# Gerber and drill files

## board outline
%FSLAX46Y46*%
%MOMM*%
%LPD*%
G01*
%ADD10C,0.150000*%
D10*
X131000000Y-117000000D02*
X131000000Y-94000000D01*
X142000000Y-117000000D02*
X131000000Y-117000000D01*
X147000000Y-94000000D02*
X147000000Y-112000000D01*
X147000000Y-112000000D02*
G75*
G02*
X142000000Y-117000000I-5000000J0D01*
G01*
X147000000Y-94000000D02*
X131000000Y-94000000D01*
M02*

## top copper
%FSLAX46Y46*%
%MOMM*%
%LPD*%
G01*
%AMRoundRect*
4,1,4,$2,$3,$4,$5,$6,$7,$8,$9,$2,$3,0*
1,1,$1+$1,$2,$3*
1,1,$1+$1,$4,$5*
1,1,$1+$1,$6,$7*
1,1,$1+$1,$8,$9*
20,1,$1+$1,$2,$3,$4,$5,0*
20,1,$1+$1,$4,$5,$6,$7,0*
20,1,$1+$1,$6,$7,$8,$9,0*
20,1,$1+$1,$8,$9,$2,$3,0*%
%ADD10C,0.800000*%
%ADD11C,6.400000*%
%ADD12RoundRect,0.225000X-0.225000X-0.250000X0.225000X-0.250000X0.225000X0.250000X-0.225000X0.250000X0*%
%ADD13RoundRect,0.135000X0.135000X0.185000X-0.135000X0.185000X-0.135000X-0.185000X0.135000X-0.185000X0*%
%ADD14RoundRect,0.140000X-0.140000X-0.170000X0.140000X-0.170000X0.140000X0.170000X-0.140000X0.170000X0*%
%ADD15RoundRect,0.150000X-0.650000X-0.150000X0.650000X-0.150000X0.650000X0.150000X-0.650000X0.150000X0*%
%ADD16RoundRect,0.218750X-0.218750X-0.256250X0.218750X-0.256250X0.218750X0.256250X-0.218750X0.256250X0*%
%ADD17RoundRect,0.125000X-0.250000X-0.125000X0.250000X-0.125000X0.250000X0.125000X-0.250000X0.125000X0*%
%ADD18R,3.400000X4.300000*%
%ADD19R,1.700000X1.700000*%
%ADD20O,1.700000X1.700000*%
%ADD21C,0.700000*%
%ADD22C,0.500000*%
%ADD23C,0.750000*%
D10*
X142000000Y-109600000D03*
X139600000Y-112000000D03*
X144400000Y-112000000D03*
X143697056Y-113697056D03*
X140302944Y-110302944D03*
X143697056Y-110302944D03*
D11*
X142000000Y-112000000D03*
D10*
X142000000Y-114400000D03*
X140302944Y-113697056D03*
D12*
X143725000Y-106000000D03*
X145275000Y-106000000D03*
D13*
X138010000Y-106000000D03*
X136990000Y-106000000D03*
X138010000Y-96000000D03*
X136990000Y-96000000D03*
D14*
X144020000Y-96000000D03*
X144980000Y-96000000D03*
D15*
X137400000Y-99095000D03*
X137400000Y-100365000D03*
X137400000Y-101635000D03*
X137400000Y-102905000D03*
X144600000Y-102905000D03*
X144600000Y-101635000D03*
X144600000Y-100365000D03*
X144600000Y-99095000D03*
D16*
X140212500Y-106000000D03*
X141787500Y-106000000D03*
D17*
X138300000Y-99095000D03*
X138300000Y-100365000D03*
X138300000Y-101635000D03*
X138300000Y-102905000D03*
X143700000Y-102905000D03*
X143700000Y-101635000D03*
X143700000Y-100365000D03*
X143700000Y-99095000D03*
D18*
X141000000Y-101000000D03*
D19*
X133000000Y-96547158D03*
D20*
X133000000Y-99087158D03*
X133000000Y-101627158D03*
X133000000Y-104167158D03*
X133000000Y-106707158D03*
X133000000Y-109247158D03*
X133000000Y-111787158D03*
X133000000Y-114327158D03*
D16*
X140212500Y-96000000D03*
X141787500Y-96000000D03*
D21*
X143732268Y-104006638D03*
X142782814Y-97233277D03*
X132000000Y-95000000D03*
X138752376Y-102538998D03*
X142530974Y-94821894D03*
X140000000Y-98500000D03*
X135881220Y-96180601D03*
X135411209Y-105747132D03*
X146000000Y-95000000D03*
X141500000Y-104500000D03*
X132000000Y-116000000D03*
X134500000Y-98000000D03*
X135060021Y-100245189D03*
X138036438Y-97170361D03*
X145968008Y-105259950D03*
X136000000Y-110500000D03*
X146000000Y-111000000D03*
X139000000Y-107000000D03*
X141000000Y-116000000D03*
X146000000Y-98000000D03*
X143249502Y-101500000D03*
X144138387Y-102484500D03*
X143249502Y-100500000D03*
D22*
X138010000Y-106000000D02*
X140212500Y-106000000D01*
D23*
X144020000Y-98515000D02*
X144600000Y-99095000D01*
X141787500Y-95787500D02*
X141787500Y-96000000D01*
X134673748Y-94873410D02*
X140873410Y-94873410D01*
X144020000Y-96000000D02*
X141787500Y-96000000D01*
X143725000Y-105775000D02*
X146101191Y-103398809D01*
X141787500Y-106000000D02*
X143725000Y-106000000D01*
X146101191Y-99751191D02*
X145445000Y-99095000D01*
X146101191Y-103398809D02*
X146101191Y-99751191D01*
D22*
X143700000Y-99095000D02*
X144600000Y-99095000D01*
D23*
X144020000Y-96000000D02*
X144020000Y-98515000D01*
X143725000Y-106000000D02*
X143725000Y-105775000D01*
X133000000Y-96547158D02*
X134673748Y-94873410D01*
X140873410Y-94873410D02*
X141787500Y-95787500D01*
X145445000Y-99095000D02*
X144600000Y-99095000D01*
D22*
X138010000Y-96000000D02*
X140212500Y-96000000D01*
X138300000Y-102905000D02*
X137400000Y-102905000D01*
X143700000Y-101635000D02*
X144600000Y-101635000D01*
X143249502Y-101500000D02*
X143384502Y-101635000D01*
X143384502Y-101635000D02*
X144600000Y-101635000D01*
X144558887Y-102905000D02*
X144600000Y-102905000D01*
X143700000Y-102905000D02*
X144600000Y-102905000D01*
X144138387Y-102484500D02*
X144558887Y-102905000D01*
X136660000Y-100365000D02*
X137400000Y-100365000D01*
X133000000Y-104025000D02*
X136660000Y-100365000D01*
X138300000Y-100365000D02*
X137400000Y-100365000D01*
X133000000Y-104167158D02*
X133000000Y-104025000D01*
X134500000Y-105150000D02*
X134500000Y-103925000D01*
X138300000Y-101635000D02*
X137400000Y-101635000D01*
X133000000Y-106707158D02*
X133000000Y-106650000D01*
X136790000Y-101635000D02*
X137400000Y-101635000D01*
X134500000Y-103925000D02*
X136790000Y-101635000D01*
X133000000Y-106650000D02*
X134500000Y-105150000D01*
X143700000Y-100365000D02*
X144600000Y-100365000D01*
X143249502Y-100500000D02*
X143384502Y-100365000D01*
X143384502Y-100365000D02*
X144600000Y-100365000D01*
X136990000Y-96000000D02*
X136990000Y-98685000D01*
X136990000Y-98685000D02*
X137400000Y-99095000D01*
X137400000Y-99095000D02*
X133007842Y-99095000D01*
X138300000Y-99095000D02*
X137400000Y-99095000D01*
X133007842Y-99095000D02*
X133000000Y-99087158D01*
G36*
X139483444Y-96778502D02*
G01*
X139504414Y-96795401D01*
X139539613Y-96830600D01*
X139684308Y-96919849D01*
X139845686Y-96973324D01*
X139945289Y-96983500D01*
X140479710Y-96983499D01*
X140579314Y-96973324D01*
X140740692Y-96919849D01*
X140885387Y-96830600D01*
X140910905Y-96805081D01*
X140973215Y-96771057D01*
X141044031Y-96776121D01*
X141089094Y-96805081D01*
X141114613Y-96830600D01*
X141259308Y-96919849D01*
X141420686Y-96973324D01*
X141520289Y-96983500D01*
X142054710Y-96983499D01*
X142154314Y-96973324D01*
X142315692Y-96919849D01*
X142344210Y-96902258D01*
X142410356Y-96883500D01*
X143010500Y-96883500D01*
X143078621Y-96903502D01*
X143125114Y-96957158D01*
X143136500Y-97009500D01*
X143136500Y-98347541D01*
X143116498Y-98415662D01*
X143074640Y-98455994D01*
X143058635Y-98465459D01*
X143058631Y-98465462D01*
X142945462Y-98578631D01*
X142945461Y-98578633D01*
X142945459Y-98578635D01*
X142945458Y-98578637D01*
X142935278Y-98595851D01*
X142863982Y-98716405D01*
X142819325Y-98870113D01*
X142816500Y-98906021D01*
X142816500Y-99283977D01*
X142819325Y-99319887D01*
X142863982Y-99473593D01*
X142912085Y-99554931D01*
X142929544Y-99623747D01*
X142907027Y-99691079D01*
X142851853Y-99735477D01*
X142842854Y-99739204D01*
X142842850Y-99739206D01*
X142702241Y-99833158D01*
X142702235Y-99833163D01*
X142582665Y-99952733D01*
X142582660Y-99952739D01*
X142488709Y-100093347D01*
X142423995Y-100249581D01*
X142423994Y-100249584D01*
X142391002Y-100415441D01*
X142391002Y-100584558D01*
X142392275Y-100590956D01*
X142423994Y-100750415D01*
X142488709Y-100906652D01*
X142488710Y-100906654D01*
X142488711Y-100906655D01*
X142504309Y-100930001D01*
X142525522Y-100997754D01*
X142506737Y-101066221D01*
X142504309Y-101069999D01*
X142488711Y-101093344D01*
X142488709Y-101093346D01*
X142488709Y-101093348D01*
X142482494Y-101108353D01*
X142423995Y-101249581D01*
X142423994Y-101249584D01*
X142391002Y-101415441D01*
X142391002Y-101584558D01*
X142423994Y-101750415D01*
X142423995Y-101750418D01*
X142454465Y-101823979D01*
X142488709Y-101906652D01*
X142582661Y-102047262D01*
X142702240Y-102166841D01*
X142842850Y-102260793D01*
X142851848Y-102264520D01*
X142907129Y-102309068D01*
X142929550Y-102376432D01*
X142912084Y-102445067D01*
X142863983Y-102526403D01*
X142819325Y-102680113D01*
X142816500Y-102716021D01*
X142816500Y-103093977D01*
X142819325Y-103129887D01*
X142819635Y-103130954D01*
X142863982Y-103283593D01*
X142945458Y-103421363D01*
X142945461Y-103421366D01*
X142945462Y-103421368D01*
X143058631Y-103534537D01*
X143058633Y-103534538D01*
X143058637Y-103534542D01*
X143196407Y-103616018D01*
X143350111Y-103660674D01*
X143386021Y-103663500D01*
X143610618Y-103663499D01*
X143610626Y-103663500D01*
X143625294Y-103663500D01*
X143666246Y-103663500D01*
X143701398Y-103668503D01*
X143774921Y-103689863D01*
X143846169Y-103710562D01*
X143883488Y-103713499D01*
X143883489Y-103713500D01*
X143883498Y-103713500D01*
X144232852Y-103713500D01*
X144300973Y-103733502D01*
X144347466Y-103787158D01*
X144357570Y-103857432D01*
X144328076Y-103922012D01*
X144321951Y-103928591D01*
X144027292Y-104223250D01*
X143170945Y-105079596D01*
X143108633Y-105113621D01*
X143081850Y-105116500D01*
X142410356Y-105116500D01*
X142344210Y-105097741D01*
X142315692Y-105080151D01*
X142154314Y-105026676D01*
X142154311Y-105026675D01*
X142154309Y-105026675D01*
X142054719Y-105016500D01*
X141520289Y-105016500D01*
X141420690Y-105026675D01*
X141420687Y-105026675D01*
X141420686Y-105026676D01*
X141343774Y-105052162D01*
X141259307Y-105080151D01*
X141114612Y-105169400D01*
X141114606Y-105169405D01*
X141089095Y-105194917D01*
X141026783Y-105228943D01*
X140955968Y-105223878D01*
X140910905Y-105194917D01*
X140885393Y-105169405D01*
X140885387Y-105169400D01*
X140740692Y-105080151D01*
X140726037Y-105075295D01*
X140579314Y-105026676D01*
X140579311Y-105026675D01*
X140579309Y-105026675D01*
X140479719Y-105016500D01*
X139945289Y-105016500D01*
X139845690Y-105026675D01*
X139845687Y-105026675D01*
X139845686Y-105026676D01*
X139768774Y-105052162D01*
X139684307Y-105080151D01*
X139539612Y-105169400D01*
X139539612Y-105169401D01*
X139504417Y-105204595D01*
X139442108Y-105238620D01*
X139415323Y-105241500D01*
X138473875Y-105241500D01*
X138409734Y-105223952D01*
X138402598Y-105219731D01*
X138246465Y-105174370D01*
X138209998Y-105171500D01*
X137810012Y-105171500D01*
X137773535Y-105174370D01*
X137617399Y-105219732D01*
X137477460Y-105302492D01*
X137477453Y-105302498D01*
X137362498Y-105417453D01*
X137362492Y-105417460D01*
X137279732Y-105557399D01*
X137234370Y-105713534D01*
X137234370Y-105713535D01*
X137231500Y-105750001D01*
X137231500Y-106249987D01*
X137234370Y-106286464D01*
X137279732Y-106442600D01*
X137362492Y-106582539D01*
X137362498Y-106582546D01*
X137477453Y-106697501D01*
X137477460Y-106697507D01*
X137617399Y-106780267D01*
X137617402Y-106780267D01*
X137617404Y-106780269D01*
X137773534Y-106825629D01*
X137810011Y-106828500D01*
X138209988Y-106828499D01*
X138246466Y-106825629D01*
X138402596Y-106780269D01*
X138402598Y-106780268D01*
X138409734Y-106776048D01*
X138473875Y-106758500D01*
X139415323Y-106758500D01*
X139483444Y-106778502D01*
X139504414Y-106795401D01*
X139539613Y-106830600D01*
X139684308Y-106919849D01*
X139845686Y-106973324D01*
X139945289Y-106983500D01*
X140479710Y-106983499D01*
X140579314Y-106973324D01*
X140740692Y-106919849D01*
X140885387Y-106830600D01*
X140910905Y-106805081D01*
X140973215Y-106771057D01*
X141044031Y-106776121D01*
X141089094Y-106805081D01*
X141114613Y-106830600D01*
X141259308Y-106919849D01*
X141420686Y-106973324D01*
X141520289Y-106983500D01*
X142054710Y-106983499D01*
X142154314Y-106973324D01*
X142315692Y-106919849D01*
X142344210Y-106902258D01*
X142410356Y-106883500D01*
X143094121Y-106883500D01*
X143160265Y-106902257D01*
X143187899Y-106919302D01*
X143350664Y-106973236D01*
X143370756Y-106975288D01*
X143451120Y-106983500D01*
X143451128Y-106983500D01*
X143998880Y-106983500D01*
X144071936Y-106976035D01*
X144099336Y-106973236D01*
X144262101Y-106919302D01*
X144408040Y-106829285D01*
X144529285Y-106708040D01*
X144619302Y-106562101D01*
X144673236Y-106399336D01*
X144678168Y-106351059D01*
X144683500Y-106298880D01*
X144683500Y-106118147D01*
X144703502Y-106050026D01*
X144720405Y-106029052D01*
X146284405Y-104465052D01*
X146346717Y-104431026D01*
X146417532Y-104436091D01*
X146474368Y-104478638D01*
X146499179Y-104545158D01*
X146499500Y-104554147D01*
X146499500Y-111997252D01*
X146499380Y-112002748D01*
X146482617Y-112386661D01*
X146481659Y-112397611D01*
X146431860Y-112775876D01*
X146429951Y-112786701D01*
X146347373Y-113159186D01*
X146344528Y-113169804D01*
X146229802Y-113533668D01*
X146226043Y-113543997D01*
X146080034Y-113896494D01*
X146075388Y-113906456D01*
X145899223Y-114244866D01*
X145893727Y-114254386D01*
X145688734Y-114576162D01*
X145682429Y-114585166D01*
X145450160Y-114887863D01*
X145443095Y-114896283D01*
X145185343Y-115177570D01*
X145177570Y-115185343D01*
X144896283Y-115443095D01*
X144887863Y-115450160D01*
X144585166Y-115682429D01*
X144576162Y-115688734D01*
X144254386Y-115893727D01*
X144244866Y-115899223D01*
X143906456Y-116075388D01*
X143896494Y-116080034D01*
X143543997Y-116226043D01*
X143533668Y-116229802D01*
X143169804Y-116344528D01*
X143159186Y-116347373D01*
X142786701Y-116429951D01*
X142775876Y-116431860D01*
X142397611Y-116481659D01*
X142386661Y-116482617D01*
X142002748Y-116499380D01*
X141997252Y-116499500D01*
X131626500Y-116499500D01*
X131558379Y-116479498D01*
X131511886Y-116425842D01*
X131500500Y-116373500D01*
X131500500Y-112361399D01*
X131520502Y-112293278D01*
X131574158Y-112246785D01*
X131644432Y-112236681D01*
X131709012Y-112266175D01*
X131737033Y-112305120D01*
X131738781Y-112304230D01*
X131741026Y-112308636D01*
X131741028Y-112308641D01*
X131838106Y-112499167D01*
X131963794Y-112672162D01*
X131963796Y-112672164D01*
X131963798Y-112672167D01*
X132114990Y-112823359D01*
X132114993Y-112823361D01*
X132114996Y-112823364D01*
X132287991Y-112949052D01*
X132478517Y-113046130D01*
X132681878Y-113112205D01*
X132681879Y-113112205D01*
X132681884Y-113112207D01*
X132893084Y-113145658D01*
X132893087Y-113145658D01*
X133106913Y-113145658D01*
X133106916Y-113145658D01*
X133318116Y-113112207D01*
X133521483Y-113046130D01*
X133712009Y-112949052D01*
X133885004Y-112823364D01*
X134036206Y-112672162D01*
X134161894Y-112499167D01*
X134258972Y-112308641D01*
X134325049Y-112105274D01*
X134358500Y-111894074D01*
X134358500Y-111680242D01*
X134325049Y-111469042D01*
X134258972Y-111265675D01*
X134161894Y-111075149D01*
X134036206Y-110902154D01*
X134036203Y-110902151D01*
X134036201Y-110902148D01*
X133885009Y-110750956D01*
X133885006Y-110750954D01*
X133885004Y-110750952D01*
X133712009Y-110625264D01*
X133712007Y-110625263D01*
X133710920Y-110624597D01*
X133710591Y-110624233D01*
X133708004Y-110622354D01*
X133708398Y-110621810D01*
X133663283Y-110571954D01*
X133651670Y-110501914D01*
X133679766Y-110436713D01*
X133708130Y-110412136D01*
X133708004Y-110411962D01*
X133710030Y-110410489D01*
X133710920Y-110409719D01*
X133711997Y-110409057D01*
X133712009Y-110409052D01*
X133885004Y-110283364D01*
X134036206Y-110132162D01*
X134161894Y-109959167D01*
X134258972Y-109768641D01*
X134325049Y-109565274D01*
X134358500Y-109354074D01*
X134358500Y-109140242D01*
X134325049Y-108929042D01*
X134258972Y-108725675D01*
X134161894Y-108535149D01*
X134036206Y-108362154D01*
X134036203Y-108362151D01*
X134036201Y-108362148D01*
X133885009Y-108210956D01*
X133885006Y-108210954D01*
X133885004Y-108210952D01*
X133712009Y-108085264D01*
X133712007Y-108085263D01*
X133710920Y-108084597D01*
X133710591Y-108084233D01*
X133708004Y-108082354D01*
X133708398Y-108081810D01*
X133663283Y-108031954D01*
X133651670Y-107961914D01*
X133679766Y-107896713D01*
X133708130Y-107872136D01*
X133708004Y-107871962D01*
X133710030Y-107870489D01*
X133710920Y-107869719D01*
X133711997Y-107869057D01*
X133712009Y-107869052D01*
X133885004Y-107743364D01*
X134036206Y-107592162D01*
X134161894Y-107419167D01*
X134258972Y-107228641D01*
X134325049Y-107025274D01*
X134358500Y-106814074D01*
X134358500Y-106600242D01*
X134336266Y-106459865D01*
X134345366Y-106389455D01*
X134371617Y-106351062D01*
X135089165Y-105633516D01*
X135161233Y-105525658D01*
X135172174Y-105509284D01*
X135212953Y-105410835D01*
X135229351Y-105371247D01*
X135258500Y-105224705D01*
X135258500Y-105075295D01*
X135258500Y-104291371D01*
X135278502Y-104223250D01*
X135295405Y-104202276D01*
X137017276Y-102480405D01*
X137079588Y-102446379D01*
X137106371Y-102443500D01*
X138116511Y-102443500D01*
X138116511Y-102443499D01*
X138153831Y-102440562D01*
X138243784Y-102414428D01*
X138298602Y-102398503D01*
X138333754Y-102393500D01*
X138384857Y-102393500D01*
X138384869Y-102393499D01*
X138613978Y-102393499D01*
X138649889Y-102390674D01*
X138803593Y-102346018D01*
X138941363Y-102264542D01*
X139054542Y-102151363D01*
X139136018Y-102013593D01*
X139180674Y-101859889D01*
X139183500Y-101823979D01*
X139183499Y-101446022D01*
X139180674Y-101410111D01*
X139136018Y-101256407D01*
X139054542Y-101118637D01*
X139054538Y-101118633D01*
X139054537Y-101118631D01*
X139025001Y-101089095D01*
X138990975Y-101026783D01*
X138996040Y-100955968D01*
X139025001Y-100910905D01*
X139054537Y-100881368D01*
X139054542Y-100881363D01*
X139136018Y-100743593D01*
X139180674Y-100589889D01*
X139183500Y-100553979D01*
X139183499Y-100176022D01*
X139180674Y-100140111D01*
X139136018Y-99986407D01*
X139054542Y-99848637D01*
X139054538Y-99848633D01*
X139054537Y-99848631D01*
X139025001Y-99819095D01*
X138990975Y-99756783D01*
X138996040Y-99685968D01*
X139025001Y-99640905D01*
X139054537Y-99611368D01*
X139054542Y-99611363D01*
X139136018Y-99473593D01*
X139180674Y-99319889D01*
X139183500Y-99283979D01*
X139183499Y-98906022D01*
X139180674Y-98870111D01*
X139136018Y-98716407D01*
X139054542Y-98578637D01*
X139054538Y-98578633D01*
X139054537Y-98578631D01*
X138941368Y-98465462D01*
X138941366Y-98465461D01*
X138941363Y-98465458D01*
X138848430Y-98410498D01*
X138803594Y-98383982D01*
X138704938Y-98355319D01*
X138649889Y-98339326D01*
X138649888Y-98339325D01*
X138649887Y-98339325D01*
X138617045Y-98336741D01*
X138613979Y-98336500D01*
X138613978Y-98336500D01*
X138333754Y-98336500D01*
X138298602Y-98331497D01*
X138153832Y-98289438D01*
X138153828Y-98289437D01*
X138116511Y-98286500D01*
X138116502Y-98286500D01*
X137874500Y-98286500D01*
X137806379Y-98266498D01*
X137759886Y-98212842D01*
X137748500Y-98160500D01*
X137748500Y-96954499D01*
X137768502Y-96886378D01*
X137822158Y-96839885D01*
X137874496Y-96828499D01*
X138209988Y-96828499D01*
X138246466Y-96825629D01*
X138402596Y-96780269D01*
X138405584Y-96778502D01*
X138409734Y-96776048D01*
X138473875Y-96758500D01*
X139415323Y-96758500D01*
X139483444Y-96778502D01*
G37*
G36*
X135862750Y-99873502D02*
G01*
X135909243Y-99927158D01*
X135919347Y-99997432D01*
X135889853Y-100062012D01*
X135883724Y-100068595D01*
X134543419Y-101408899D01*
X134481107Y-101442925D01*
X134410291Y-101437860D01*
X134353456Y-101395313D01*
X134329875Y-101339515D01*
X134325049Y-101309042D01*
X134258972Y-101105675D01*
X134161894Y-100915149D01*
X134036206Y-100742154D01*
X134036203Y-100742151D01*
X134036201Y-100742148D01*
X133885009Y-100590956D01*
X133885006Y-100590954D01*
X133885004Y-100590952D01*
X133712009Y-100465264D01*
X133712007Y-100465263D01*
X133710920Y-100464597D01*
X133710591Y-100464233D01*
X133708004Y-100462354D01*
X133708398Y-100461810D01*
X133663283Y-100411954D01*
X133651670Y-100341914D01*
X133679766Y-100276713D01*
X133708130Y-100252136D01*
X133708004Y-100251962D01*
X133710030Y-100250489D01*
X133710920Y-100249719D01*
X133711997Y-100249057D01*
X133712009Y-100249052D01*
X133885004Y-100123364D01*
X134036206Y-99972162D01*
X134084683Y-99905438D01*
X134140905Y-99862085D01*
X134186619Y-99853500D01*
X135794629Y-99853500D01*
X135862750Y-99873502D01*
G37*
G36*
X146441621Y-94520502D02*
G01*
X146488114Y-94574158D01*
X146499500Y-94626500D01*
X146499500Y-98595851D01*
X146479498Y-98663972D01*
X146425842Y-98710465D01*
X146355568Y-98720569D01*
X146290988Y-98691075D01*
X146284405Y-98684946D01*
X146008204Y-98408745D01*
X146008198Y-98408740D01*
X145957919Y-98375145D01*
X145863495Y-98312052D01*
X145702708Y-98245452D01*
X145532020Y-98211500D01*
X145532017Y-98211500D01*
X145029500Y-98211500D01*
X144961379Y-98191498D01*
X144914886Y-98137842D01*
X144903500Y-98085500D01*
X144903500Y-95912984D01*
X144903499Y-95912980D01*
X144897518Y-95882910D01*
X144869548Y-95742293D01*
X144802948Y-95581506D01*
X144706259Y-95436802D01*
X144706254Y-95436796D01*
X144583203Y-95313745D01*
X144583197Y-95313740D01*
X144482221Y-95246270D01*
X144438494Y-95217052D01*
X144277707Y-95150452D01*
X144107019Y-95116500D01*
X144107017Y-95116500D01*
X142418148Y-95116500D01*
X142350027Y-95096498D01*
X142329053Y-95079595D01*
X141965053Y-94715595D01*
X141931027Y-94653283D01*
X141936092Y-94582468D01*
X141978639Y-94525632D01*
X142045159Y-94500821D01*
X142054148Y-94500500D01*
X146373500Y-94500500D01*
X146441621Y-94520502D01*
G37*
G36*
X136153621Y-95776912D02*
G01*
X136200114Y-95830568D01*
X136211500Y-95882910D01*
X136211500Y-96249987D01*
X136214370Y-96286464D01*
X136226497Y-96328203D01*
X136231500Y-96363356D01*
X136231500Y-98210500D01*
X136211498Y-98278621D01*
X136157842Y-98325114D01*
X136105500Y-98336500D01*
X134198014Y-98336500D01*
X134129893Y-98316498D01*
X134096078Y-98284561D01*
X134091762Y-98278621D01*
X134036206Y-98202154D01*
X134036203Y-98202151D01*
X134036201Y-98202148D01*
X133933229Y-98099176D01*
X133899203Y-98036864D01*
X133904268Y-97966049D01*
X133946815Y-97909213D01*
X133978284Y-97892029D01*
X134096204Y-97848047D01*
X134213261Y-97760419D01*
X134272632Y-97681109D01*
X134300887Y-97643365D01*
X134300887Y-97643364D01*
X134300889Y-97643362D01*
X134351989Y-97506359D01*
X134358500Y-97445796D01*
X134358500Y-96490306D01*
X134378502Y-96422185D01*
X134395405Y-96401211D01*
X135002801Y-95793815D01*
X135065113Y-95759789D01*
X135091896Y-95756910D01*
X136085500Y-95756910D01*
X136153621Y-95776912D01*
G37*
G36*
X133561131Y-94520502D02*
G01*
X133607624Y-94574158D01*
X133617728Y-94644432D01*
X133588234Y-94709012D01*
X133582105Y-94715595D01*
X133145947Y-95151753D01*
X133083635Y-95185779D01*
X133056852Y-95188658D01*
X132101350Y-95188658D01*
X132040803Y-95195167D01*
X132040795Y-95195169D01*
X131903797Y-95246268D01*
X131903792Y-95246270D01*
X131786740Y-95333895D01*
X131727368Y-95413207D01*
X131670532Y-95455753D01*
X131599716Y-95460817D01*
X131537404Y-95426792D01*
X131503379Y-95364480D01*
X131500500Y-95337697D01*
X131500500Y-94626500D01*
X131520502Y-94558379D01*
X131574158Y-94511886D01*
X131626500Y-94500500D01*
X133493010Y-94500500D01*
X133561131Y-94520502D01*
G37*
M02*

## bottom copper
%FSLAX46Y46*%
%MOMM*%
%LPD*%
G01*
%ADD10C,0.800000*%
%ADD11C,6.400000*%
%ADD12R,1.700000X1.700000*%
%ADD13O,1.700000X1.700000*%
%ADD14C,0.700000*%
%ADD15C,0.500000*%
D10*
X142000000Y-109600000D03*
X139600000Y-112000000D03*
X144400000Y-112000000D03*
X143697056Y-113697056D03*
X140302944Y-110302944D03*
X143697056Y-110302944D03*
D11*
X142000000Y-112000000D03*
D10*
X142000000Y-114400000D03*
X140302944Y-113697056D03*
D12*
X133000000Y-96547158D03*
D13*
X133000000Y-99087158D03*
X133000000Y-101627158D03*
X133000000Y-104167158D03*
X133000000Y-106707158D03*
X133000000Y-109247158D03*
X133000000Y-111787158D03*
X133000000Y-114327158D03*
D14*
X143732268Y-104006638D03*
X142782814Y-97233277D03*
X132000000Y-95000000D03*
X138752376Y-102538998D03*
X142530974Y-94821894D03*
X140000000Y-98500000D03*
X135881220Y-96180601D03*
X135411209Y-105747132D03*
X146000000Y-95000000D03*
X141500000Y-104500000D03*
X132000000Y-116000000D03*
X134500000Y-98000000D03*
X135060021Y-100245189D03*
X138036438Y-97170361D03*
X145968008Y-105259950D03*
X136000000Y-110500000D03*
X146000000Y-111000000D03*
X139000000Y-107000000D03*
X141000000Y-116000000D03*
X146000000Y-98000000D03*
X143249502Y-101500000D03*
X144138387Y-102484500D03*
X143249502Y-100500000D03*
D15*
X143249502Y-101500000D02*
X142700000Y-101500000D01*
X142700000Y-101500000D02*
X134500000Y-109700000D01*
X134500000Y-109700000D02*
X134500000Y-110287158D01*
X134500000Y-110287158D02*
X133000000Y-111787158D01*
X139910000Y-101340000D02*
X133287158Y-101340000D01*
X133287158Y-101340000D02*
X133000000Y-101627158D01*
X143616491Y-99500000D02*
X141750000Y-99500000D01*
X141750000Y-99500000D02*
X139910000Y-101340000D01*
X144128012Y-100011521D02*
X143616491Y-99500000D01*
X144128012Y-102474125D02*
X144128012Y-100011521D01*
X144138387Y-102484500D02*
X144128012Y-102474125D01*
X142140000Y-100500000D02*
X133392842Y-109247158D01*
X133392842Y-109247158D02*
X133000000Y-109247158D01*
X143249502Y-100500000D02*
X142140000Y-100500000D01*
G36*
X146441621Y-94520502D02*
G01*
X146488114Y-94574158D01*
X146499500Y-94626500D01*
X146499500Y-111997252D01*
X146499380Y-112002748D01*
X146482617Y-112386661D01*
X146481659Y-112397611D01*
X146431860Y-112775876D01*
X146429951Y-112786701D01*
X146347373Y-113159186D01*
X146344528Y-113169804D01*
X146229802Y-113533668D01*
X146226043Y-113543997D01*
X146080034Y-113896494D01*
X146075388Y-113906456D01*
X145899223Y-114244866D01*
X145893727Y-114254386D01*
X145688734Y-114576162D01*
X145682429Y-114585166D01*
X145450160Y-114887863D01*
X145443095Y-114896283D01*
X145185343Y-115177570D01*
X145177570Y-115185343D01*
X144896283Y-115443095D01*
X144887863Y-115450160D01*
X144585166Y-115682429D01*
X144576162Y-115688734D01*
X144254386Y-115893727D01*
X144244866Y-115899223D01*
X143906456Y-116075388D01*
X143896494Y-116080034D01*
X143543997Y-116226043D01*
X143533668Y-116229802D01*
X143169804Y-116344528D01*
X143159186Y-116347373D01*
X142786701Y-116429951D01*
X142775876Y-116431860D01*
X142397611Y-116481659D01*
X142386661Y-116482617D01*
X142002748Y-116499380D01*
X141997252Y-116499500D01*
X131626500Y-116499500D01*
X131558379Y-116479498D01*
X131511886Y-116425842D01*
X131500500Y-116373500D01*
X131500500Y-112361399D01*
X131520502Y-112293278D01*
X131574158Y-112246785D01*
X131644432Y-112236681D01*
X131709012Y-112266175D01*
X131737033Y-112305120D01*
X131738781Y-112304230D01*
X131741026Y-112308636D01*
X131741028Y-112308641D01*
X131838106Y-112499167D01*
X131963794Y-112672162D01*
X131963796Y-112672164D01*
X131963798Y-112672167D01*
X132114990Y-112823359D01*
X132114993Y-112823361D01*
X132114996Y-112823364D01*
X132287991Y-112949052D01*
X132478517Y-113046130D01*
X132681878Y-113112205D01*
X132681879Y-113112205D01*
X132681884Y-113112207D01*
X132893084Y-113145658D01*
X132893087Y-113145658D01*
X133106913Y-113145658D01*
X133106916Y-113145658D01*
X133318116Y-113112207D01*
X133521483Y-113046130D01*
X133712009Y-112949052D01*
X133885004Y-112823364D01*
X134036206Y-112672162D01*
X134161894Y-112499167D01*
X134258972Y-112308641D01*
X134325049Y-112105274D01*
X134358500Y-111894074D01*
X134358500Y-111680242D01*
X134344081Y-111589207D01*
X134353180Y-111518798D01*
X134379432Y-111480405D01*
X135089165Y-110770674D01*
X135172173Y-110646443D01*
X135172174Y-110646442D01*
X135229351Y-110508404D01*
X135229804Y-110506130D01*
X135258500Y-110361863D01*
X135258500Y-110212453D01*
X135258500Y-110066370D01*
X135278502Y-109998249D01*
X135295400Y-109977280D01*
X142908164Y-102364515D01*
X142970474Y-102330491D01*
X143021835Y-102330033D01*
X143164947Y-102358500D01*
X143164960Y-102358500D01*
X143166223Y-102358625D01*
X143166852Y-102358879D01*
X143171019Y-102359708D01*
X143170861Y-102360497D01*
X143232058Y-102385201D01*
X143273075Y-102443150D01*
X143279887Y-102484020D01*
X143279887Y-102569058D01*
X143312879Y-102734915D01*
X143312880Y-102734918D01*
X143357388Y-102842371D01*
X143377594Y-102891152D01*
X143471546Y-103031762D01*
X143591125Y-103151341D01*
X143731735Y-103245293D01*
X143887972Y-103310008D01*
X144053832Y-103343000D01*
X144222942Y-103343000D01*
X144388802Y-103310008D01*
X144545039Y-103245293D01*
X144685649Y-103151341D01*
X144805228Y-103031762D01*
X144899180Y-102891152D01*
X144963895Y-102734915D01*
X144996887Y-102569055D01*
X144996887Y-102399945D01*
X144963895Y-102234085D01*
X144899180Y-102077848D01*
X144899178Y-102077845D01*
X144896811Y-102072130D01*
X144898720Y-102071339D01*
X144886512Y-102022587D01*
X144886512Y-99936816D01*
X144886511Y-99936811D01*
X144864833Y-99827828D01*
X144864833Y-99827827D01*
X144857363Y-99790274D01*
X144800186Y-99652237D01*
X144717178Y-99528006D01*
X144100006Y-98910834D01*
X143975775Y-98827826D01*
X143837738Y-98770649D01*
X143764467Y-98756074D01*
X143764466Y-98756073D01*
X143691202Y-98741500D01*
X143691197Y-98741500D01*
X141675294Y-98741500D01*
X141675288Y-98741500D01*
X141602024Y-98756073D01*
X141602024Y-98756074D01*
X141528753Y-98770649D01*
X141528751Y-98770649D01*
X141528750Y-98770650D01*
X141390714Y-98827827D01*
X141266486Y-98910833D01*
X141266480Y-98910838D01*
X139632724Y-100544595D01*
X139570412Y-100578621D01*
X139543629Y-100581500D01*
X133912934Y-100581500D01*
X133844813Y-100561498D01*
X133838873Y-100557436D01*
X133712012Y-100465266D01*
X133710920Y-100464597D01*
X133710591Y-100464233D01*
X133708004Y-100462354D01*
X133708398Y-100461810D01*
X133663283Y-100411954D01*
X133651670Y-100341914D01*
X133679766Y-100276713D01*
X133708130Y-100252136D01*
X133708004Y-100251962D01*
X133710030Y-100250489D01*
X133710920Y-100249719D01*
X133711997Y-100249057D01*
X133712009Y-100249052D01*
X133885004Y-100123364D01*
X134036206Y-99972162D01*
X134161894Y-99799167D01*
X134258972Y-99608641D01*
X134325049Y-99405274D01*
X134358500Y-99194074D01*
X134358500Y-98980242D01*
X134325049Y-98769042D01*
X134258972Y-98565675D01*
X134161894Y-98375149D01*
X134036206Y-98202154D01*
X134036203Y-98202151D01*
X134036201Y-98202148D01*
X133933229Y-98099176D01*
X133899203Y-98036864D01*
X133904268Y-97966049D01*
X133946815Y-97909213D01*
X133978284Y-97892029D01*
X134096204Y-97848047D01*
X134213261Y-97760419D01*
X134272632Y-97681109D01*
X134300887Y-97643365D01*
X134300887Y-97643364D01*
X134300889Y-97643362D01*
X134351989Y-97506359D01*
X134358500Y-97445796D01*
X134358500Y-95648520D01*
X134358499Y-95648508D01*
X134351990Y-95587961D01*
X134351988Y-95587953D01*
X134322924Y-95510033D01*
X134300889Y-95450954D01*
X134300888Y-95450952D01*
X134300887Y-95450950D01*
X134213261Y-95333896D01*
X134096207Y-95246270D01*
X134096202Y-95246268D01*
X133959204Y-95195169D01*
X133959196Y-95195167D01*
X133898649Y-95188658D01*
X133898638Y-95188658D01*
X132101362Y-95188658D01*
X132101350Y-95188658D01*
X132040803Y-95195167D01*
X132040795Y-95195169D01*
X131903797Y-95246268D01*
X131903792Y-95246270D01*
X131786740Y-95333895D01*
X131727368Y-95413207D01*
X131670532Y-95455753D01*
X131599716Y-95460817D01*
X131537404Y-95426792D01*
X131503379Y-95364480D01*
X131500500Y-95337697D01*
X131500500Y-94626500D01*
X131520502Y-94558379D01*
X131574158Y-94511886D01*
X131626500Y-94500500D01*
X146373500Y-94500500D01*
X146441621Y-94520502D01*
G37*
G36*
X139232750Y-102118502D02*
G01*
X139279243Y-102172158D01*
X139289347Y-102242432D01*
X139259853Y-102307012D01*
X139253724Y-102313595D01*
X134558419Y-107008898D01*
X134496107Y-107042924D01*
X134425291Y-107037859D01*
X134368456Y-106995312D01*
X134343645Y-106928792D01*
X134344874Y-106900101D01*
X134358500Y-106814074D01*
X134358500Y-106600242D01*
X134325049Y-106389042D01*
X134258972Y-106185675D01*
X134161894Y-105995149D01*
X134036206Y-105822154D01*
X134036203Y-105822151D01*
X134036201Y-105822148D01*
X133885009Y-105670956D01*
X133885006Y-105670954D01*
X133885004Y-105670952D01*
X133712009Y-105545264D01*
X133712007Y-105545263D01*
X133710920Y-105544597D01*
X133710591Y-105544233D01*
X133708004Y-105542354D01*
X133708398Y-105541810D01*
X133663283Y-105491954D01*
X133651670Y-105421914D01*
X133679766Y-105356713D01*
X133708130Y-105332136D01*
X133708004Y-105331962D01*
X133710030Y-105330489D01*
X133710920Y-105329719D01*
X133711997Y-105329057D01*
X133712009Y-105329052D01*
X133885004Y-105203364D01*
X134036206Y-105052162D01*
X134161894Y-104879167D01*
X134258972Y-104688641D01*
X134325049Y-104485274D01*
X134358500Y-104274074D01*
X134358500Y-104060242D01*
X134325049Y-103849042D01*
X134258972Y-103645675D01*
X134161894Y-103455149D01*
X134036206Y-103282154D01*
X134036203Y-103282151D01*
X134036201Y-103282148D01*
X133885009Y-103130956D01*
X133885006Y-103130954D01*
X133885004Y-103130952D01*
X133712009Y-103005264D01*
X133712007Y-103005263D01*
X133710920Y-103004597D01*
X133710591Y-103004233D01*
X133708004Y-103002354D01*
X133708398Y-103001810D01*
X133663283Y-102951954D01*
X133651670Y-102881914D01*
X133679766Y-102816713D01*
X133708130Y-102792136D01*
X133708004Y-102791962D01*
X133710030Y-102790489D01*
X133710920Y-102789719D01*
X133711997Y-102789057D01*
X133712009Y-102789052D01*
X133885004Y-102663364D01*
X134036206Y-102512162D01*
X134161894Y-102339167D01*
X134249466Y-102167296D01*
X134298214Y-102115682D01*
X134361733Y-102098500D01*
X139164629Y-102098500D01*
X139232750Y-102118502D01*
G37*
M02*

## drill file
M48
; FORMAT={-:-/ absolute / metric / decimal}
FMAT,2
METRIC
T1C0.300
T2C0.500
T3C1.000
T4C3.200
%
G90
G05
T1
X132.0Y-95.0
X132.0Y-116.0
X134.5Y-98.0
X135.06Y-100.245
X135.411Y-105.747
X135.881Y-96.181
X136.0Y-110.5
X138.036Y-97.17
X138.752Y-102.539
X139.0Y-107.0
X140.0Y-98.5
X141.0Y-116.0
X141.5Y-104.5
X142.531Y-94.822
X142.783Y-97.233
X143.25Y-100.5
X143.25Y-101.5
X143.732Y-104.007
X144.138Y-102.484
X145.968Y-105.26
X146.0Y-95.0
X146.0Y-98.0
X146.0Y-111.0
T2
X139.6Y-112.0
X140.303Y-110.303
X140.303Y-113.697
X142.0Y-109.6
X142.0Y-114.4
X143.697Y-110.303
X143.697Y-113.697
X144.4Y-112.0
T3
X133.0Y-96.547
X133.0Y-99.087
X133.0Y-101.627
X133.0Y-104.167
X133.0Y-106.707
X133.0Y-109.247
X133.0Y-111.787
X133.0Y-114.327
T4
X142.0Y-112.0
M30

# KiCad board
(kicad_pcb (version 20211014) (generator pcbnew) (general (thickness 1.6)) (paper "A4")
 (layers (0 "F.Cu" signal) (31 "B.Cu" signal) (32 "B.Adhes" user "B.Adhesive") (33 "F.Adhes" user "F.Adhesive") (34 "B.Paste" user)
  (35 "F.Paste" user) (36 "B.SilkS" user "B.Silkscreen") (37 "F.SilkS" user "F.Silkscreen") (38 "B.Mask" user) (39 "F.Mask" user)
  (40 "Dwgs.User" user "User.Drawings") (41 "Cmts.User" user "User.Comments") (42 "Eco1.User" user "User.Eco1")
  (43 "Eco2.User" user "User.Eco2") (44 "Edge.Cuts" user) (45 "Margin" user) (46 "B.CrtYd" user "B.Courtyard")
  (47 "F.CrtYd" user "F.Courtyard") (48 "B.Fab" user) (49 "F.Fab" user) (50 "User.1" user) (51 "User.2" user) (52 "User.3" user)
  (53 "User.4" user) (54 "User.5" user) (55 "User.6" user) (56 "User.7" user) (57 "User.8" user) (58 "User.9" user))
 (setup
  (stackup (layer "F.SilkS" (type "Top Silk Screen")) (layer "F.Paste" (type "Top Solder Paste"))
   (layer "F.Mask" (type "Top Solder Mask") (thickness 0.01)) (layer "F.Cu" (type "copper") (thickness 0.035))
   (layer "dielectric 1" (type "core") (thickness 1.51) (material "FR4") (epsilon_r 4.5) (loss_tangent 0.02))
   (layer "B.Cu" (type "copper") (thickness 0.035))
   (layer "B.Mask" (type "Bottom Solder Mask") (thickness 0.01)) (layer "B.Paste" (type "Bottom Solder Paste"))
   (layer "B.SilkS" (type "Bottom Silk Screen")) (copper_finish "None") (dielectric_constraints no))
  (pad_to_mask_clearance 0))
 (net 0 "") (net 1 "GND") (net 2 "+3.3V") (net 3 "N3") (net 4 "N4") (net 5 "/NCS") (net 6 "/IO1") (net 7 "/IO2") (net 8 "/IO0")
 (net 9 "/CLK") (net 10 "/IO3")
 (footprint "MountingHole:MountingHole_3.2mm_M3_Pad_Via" (layer "F.Cu") (at 142 112)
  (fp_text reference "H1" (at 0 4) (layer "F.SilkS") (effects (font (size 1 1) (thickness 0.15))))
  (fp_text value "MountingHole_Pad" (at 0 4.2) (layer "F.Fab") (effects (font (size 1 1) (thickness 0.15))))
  (pad "1" thru_hole circle (at 0 -2.4) (size 0.8 0.8) (drill 0.5) (layers *.Cu *.Mask) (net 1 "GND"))
  (pad "1" thru_hole circle (at -2.4 0) (size 0.8 0.8) (drill 0.5) (layers *.Cu *.Mask) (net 1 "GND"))
  (pad "1" thru_hole circle (at 2.4 0) (size 0.8 0.8) (drill 0.5) (layers *.Cu *.Mask) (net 1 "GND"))
  (pad "1" thru_hole circle (at 1.697056 1.697056) (size 0.8 0.8) (drill 0.5) (layers *.Cu *.Mask) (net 1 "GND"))
  (pad "1" thru_hole circle (at -1.697056 -1.697056) (size 0.8 0.8) (drill 0.5) (layers *.Cu *.Mask) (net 1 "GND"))
  (pad "1" thru_hole circle (at 1.697056 -1.697056) (size 0.8 0.8) (drill 0.5) (layers *.Cu *.Mask) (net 1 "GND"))
  (pad "1" thru_hole circle (at 0 0) (size 6.4 6.4) (drill 3.2) (layers *.Cu *.Mask) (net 1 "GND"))
  (pad "1" thru_hole circle (at 0 2.4) (size 0.8 0.8) (drill 0.5) (layers *.Cu *.Mask) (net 1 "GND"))
  (pad "1" thru_hole circle (at -1.697056 1.697056) (size 0.8 0.8) (drill 0.5) (layers *.Cu *.Mask) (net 1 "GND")))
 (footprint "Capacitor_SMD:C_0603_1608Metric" (layer "F.Cu") (at 144.5 106)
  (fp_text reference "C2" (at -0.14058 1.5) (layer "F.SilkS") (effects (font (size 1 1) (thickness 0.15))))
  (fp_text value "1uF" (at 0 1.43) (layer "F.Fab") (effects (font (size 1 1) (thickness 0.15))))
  (pad "1" smd roundrect (at -0.775 0) (size 0.9 0.95) (layers "F.Cu" "F.Paste" "F.Mask") (roundrect_rratio 0.25) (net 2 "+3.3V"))
  (pad "2" smd roundrect (at 0.775 0) (size 0.9 0.95) (layers "F.Cu" "F.Paste" "F.Mask") (roundrect_rratio 0.25) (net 1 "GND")))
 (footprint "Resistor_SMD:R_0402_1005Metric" (layer "F.Cu") (at 137.5 106 180)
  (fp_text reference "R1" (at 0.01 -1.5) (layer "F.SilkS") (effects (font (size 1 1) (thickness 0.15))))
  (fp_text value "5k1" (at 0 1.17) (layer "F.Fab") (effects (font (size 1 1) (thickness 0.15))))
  (pad "1" smd roundrect (at -0.51 0 180) (size 0.54 0.64) (layers "F.Cu" "F.Paste" "F.Mask") (roundrect_rratio 0.25) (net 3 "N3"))
  (pad "2" smd roundrect (at 0.51 0 180) (size 0.54 0.64) (layers "F.Cu" "F.Paste" "F.Mask") (roundrect_rratio 0.25) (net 1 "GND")))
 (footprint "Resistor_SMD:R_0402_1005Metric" (layer "F.Cu") (at 137.5 96 180)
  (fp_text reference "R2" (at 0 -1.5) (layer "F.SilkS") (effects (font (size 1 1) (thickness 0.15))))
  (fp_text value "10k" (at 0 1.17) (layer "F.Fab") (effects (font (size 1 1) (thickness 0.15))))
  (pad "1" smd roundrect (at -0.51 0 180) (size 0.54 0.64) (layers "F.Cu" "F.Paste" "F.Mask") (roundrect_rratio 0.25) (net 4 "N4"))
  (pad "2" smd roundrect (at 0.51 0 180) (size 0.54 0.64) (layers "F.Cu" "F.Paste" "F.Mask") (roundrect_rratio 0.25) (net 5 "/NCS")))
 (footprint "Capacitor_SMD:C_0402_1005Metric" (layer "F.Cu") (at 144.5 96)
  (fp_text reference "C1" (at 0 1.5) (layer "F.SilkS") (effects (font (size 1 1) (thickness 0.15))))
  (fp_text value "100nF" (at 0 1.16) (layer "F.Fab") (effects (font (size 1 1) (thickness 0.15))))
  (pad "1" smd roundrect (at -0.48 0) (size 0.56 0.62) (layers "F.Cu" "F.Paste" "F.Mask") (roundrect_rratio 0.25) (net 2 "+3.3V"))
  (pad "2" smd roundrect (at 0.48 0) (size 0.56 0.62) (layers "F.Cu" "F.Paste" "F.Mask") (roundrect_rratio 0.25) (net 1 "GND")))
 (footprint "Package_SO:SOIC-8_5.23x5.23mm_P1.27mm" (layer "F.Cu") (at 141 101)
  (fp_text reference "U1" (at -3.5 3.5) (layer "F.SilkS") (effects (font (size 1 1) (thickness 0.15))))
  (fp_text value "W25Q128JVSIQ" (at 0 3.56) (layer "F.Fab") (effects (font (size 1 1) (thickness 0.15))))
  (pad "1" smd roundrect (at -3.6 -1.905) (size 1.6 0.6) (layers "F.Cu" "F.Paste" "F.Mask") (roundrect_rratio 0.25) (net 5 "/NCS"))
  (pad "2" smd roundrect (at -3.6 -0.635) (size 1.6 0.6) (layers "F.Cu" "F.Paste" "F.Mask") (roundrect_rratio 0.25) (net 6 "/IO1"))
  (pad "3" smd roundrect (at -3.6 0.635) (size 1.6 0.6) (layers "F.Cu" "F.Paste" "F.Mask") (roundrect_rratio 0.25) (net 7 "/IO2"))
  (pad "4" smd roundrect (at -3.6 1.905) (size 1.6 0.6) (layers "F.Cu" "F.Paste" "F.Mask") (roundrect_rratio 0.25) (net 1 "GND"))
  (pad "5" smd roundrect (at 3.6 1.905) (size 1.6 0.6) (layers "F.Cu" "F.Paste" "F.Mask") (roundrect_rratio 0.25) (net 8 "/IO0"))
  (pad "6" smd roundrect (at 3.6 0.635) (size 1.6 0.6) (layers "F.Cu" "F.Paste" "F.Mask") (roundrect_rratio 0.25) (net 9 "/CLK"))
  (pad "7" smd roundrect (at 3.6 -0.635) (size 1.6 0.6) (layers "F.Cu" "F.Paste" "F.Mask") (roundrect_rratio 0.25) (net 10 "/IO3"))
  (pad "8" smd roundrect (at 3.6 -1.905) (size 1.6 0.6) (layers "F.Cu" "F.Paste" "F.Mask") (roundrect_rratio 0.25) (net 2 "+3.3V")))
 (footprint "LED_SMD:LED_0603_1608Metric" (layer "F.Cu") (at 141 106)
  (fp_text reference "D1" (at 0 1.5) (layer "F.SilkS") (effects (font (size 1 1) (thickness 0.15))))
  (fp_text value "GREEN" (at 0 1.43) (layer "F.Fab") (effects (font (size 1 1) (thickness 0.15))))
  (pad "1" smd roundrect (at -0.7875 0) (size 0.875 0.95) (layers "F.Cu" "F.Paste" "F.Mask") (roundrect_rratio 0.25) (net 3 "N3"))
  (pad "2" smd roundrect (at 0.7875 0) (size 0.875 0.95) (layers "F.Cu" "F.Paste" "F.Mask") (roundrect_rratio 0.25) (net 2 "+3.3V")))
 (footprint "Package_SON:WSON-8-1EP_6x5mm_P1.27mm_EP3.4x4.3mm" (layer "F.Cu") (at 141 101)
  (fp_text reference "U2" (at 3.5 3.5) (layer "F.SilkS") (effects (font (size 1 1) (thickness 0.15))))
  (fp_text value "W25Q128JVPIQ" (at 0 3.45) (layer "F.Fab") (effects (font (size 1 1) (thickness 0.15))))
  (pad "" smd roundrect (at -0.85 1.075) (size 1.37 1.73) (layers "F.Paste") (roundrect_rratio 0.182482))
  (pad "" smd roundrect (at 0.85 -1.075) (size 1.37 1.73) (layers "F.Paste") (roundrect_rratio 0.182482))
  (pad "" smd roundrect (at 0.85 1.075) (size 1.37 1.73) (layers "F.Paste") (roundrect_rratio 0.182482))
  (pad "" smd roundrect (at -0.85 -1.075) (size 1.37 1.73) (layers "F.Paste") (roundrect_rratio 0.182482))
  (pad "1" smd roundrect (at -2.7 -1.905) (size 0.75 0.5) (layers "F.Cu" "F.Paste" "F.Mask") (roundrect_rratio 0.25) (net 5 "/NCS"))
  (pad "2" smd roundrect (at -2.7 -0.635) (size 0.75 0.5) (layers "F.Cu" "F.Paste" "F.Mask") (roundrect_rratio 0.25) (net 6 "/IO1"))
  (pad "3" smd roundrect (at -2.7 0.635) (size 0.75 0.5) (layers "F.Cu" "F.Paste" "F.Mask") (roundrect_rratio 0.25) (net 7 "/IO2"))
  (pad "4" smd roundrect (at -2.7 1.905) (size 0.75 0.5) (layers "F.Cu" "F.Paste" "F.Mask") (roundrect_rratio 0.25) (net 1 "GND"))
  (pad "5" smd roundrect (at 2.7 1.905) (size 0.75 0.5) (layers "F.Cu" "F.Paste" "F.Mask") (roundrect_rratio 0.25) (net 8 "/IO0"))
  (pad "6" smd roundrect (at 2.7 0.635) (size 0.75 0.5) (layers "F.Cu" "F.Paste" "F.Mask") (roundrect_rratio 0.25) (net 9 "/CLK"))
  (pad "7" smd roundrect (at 2.7 -0.635) (size 0.75 0.5) (layers "F.Cu" "F.Paste" "F.Mask") (roundrect_rratio 0.25) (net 10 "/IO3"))
  (pad "8" smd roundrect (at 2.7 -1.905) (size 0.75 0.5) (layers "F.Cu" "F.Paste" "F.Mask") (roundrect_rratio 0.25) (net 2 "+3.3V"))
  (pad "9" smd rect (at 0 0) (size 3.4 4.3) (layers "F.Cu" "F.Mask") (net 1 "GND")))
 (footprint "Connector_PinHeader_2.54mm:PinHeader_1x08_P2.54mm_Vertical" (layer "F.Cu") (at 133 96.547158)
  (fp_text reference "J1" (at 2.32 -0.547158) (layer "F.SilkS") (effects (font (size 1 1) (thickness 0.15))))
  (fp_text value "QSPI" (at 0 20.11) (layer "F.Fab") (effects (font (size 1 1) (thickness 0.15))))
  (pad "1" thru_hole rect (at 0 0) (size 1.7 1.7) (drill 1) (layers *.Cu *.Mask) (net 2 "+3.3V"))
  (pad "2" thru_hole oval (at 0 2.54) (size 1.7 1.7) (drill 1) (layers *.Cu *.Mask) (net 5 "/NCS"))
  (pad "3" thru_hole oval (at 0 5.08) (size 1.7 1.7) (drill 1) (layers *.Cu *.Mask) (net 8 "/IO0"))
  (pad "4" thru_hole oval (at 0 7.62) (size 1.7 1.7) (drill 1) (layers *.Cu *.Mask) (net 6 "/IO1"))
  (pad "5" thru_hole oval (at 0 10.16) (size 1.7 1.7) (drill 1) (layers *.Cu *.Mask) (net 7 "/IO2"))
  (pad "6" thru_hole oval (at 0 12.7) (size 1.7 1.7) (drill 1) (layers *.Cu *.Mask) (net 10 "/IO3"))
  (pad "7" thru_hole oval (at 0 15.24) (size 1.7 1.7) (drill 1) (layers *.Cu *.Mask) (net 9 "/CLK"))
  (pad "8" thru_hole oval (at 0 17.78) (size 1.7 1.7) (drill 1) (layers *.Cu *.Mask) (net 1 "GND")))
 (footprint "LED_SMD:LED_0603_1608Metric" (layer "F.Cu") (at 141 96)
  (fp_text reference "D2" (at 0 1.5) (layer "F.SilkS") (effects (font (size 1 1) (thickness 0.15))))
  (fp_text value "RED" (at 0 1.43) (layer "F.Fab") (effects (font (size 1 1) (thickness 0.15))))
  (pad "1" smd roundrect (at -0.7875 0) (size 0.875 0.95) (layers "F.Cu" "F.Paste" "F.Mask") (roundrect_rratio 0.25) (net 4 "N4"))
  (pad "2" smd roundrect (at 0.7875 0) (size 0.875 0.95) (layers "F.Cu" "F.Paste" "F.Mask") (roundrect_rratio 0.25) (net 2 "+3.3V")))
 (gr_line (start 131 117) (end 131 94) (layer "Edge.Cuts") (width 0.15))
 (gr_line (start 142 117) (end 131 117) (layer "Edge.Cuts") (width 0.15))
 (gr_line (start 147 94) (end 147 112) (layer "Edge.Cuts") (width 0.15))
 (gr_arc (start 147 112) (mid 145.535534 115.535534) (end 142 117) (layer "Edge.Cuts") (width 0.15))
 (gr_line (start 147 94) (end 131 94) (layer "Edge.Cuts") (width 0.15))
 (segment (start 138.01 106) (end 140.2125 106) (width 0.5) (layer "F.Cu") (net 3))
 (segment (start 144.02 98.515) (end 144.6 99.095) (width 0.75) (layer "F.Cu") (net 2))
 (segment (start 141.7875 95.7875) (end 141.7875 96) (width 0.75) (layer "F.Cu") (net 2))
 (segment (start 134.673748 94.87341) (end 140.87341 94.87341) (width 0.75) (layer "F.Cu") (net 2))
 (segment (start 144.02 96) (end 141.7875 96) (width 0.75) (layer "F.Cu") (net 2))
 (segment (start 143.725 105.775) (end 146.101191 103.398809) (width 0.75) (layer "F.Cu") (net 2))
 (segment (start 141.7875 106) (end 143.725 106) (width 0.75) (layer "F.Cu") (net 2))
 (segment (start 146.101191 99.751191) (end 145.445 99.095) (width 0.75) (layer "F.Cu") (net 2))
 (segment (start 146.101191 103.398809) (end 146.101191 99.751191) (width 0.75) (layer "F.Cu") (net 2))
 (segment (start 143.7 99.095) (end 144.6 99.095) (width 0.5) (layer "F.Cu") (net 2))
 (segment (start 144.02 96) (end 144.02 98.515) (width 0.75) (layer "F.Cu") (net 2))
 (segment (start 143.725 106) (end 143.725 105.775) (width 0.75) (layer "F.Cu") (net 2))
 (segment (start 133 96.547158) (end 134.673748 94.87341) (width 0.75) (layer "F.Cu") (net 2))
 (segment (start 140.87341 94.87341) (end 141.7875 95.7875) (width 0.75) (layer "F.Cu") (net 2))
 (segment (start 145.445 99.095) (end 144.6 99.095) (width 0.75) (layer "F.Cu") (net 2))
 (segment (start 138.01 96) (end 140.2125 96) (width 0.5) (layer "F.Cu") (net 4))
 (segment (start 138.3 102.905) (end 137.4 102.905) (width 0.5) (layer "F.Cu") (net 1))
 (via (at 143.732268 104.006638) (size 0.7) (drill 0.3) (layers "F.Cu" "B.Cu") (free) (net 1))
 (via (at 142.782814 97.233277) (size 0.7) (drill 0.3) (layers "F.Cu" "B.Cu") (free) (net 1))
 (via (at 132 95) (size 0.7) (drill 0.3) (layers "F.Cu" "B.Cu") (free) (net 1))
 (via (at 138.752376 102.538998) (size 0.7) (drill 0.3) (layers "F.Cu" "B.Cu") (free) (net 1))
 (via (at 142.530974 94.821894) (size 0.7) (drill 0.3) (layers "F.Cu" "B.Cu") (free) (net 1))
 (via (at 140 98.5) (size 0.7) (drill 0.3) (layers "F.Cu" "B.Cu") (free) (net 1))
 (via (at 135.88122 96.180601) (size 0.7) (drill 0.3) (layers "F.Cu" "B.Cu") (free) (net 1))
 (via (at 135.411209 105.747132) (size 0.7) (drill 0.3) (layers "F.Cu" "B.Cu") (free) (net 1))
 (via (at 146 95) (size 0.7) (drill 0.3) (layers "F.Cu" "B.Cu") (free) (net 1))
 (via (at 141.5 104.5) (size 0.7) (drill 0.3) (layers "F.Cu" "B.Cu") (free) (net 1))
 (via (at 132 116) (size 0.7) (drill 0.3) (layers "F.Cu" "B.Cu") (free) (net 1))
 (via (at 134.5 98) (size 0.7) (drill 0.3) (layers "F.Cu" "B.Cu") (free) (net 1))
 (via (at 135.060021 100.245189) (size 0.7) (drill 0.3) (layers "F.Cu" "B.Cu") (free) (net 1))
 (via (at 138.036438 97.170361) (size 0.7) (drill 0.3) (layers "F.Cu" "B.Cu") (free) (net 1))
 (via (at 145.968008 105.25995) (size 0.7) (drill 0.3) (layers "F.Cu" "B.Cu") (free) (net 1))
 (via (at 136 110.5) (size 0.7) (drill 0.3) (layers "F.Cu" "B.Cu") (free) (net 1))
 (via (at 146 111) (size 0.7) (drill 0.3) (layers "F.Cu" "B.Cu") (free) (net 1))
 (via (at 139 107) (size 0.7) (drill 0.3) (layers "F.Cu" "B.Cu") (free) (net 1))
 (via (at 141 116) (size 0.7) (drill 0.3) (layers "F.Cu" "B.Cu") (free) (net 1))
 (via (at 146 98) (size 0.7) (drill 0.3) (layers "F.Cu" "B.Cu") (free) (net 1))
 (segment (start 143.7 101.635) (end 144.6 101.635) (width 0.5) (layer "F.Cu") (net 9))
 (segment (start 143.249502 101.5) (end 143.384502 101.635) (width 0.5) (layer "F.Cu") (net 9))
 (segment (start 143.384502 101.635) (end 144.6 101.635) (width 0.5) (layer "F.Cu") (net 9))
 (via (at 143.249502 101.5) (size 0.7) (drill 0.3) (layers "F.Cu" "B.Cu") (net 9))
 (segment (start 143.249502 101.5) (end 142.7 101.5) (width 0.5) (layer "B.Cu") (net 9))
 (segment (start 142.7 101.5) (end 134.5 109.7) (width 0.5) (layer "B.Cu") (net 9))
 (segment (start 134.5 109.7) (end 134.5 110.287158) (width 0.5) (layer "B.Cu") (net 9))
 (segment (start 134.5 110.287158) (end 133 111.787158) (width 0.5) (layer "B.Cu") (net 9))
 (segment (start 144.558887 102.905) (end 144.6 102.905) (width 0.5) (layer "F.Cu") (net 8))
 (segment (start 143.7 102.905) (end 144.6 102.905) (width 0.5) (layer "F.Cu") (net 8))
 (segment (start 144.138387 102.4845) (end 144.558887 102.905) (width 0.5) (layer "F.Cu") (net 8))
 (via (at 144.138387 102.4845) (size 0.7) (drill 0.3) (layers "F.Cu" "B.Cu") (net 8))
 (segment (start 139.91 101.34) (end 133.287158 101.34) (width 0.5) (layer "B.Cu") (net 8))
 (segment (start 133.287158 101.34) (end 133 101.627158) (width 0.5) (layer "B.Cu") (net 8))
 (segment (start 143.616491 99.5) (end 141.75 99.5) (width 0.5) (layer "B.Cu") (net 8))
 (segment (start 141.75 99.5) (end 139.91 101.34) (width 0.5) (layer "B.Cu") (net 8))
 (segment (start 144.128012 100.011521) (end 143.616491 99.5) (width 0.5) (layer "B.Cu") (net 8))
 (segment (start 144.128012 102.474125) (end 144.128012 100.011521) (width 0.5) (layer "B.Cu") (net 8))
 (segment (start 144.138387 102.4845) (end 144.128012 102.474125) (width 0.5) (layer "B.Cu") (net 8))
 (segment (start 136.66 100.365) (end 137.4 100.365) (width 0.5) (layer "F.Cu") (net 6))
 (segment (start 133 104.025) (end 136.66 100.365) (width 0.5) (layer "F.Cu") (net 6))
 (segment (start 138.3 100.365) (end 137.4 100.365) (width 0.5) (layer "F.Cu") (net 6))
 (segment (start 133 104.167158) (end 133 104.025) (width 0.5) (layer "F.Cu") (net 6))
 (segment (start 134.5 105.15) (end 134.5 103.925) (width 0.5) (layer "F.Cu") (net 7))
 (segment (start 138.3 101.635) (end 137.4 101.635) (width 0.5) (layer "F.Cu") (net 7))
 (segment (start 133 106.707158) (end 133 106.65) (width 0.5) (layer "F.Cu") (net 7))
 (segment (start 136.79 101.635) (end 137.4 101.635) (width 0.5) (layer "F.Cu") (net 7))
 (segment (start 134.5 103.925) (end 136.79 101.635) (width 0.5) (layer "F.Cu") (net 7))
 (segment (start 133 106.65) (end 134.5 105.15) (width 0.5) (layer "F.Cu") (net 7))
 (segment (start 143.7 100.365) (end 144.6 100.365) (width 0.5) (layer "F.Cu") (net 10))
 (segment (start 143.249502 100.5) (end 143.384502 100.365) (width 0.5) (layer "F.Cu") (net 10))
 (segment (start 143.384502 100.365) (end 144.6 100.365) (width 0.5) (layer "F.Cu") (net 10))
 (via (at 143.249502 100.5) (size 0.7) (drill 0.3) (layers "F.Cu" "B.Cu") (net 10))
 (segment (start 142.14 100.5) (end 133.392842 109.247158) (width 0.5) (layer "B.Cu") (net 10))
 (segment (start 133.392842 109.247158) (end 133 109.247158) (width 0.5) (layer "B.Cu") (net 10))
 (segment (start 143.249502 100.5) (end 142.14 100.5) (width 0.5) (layer "B.Cu") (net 10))
 (segment (start 136.99 96) (end 136.99 98.685) (width 0.5) (layer "F.Cu") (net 5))
 (segment (start 136.99 98.685) (end 137.4 99.095) (width 0.5) (layer "F.Cu") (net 5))
 (segment (start 137.4 99.095) (end 133.007842 99.095) (width 0.5) (layer "F.Cu") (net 5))
 (segment (start 138.3 99.095) (end 137.4 99.095) (width 0.5) (layer "F.Cu") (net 5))
 (segment (start 133.007842 99.095) (end 133 99.087158) (width 0.5) (layer "F.Cu") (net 5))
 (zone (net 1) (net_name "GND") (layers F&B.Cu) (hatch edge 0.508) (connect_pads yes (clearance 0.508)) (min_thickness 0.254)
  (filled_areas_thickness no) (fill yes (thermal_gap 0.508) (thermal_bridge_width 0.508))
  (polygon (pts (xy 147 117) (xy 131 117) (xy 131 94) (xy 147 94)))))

